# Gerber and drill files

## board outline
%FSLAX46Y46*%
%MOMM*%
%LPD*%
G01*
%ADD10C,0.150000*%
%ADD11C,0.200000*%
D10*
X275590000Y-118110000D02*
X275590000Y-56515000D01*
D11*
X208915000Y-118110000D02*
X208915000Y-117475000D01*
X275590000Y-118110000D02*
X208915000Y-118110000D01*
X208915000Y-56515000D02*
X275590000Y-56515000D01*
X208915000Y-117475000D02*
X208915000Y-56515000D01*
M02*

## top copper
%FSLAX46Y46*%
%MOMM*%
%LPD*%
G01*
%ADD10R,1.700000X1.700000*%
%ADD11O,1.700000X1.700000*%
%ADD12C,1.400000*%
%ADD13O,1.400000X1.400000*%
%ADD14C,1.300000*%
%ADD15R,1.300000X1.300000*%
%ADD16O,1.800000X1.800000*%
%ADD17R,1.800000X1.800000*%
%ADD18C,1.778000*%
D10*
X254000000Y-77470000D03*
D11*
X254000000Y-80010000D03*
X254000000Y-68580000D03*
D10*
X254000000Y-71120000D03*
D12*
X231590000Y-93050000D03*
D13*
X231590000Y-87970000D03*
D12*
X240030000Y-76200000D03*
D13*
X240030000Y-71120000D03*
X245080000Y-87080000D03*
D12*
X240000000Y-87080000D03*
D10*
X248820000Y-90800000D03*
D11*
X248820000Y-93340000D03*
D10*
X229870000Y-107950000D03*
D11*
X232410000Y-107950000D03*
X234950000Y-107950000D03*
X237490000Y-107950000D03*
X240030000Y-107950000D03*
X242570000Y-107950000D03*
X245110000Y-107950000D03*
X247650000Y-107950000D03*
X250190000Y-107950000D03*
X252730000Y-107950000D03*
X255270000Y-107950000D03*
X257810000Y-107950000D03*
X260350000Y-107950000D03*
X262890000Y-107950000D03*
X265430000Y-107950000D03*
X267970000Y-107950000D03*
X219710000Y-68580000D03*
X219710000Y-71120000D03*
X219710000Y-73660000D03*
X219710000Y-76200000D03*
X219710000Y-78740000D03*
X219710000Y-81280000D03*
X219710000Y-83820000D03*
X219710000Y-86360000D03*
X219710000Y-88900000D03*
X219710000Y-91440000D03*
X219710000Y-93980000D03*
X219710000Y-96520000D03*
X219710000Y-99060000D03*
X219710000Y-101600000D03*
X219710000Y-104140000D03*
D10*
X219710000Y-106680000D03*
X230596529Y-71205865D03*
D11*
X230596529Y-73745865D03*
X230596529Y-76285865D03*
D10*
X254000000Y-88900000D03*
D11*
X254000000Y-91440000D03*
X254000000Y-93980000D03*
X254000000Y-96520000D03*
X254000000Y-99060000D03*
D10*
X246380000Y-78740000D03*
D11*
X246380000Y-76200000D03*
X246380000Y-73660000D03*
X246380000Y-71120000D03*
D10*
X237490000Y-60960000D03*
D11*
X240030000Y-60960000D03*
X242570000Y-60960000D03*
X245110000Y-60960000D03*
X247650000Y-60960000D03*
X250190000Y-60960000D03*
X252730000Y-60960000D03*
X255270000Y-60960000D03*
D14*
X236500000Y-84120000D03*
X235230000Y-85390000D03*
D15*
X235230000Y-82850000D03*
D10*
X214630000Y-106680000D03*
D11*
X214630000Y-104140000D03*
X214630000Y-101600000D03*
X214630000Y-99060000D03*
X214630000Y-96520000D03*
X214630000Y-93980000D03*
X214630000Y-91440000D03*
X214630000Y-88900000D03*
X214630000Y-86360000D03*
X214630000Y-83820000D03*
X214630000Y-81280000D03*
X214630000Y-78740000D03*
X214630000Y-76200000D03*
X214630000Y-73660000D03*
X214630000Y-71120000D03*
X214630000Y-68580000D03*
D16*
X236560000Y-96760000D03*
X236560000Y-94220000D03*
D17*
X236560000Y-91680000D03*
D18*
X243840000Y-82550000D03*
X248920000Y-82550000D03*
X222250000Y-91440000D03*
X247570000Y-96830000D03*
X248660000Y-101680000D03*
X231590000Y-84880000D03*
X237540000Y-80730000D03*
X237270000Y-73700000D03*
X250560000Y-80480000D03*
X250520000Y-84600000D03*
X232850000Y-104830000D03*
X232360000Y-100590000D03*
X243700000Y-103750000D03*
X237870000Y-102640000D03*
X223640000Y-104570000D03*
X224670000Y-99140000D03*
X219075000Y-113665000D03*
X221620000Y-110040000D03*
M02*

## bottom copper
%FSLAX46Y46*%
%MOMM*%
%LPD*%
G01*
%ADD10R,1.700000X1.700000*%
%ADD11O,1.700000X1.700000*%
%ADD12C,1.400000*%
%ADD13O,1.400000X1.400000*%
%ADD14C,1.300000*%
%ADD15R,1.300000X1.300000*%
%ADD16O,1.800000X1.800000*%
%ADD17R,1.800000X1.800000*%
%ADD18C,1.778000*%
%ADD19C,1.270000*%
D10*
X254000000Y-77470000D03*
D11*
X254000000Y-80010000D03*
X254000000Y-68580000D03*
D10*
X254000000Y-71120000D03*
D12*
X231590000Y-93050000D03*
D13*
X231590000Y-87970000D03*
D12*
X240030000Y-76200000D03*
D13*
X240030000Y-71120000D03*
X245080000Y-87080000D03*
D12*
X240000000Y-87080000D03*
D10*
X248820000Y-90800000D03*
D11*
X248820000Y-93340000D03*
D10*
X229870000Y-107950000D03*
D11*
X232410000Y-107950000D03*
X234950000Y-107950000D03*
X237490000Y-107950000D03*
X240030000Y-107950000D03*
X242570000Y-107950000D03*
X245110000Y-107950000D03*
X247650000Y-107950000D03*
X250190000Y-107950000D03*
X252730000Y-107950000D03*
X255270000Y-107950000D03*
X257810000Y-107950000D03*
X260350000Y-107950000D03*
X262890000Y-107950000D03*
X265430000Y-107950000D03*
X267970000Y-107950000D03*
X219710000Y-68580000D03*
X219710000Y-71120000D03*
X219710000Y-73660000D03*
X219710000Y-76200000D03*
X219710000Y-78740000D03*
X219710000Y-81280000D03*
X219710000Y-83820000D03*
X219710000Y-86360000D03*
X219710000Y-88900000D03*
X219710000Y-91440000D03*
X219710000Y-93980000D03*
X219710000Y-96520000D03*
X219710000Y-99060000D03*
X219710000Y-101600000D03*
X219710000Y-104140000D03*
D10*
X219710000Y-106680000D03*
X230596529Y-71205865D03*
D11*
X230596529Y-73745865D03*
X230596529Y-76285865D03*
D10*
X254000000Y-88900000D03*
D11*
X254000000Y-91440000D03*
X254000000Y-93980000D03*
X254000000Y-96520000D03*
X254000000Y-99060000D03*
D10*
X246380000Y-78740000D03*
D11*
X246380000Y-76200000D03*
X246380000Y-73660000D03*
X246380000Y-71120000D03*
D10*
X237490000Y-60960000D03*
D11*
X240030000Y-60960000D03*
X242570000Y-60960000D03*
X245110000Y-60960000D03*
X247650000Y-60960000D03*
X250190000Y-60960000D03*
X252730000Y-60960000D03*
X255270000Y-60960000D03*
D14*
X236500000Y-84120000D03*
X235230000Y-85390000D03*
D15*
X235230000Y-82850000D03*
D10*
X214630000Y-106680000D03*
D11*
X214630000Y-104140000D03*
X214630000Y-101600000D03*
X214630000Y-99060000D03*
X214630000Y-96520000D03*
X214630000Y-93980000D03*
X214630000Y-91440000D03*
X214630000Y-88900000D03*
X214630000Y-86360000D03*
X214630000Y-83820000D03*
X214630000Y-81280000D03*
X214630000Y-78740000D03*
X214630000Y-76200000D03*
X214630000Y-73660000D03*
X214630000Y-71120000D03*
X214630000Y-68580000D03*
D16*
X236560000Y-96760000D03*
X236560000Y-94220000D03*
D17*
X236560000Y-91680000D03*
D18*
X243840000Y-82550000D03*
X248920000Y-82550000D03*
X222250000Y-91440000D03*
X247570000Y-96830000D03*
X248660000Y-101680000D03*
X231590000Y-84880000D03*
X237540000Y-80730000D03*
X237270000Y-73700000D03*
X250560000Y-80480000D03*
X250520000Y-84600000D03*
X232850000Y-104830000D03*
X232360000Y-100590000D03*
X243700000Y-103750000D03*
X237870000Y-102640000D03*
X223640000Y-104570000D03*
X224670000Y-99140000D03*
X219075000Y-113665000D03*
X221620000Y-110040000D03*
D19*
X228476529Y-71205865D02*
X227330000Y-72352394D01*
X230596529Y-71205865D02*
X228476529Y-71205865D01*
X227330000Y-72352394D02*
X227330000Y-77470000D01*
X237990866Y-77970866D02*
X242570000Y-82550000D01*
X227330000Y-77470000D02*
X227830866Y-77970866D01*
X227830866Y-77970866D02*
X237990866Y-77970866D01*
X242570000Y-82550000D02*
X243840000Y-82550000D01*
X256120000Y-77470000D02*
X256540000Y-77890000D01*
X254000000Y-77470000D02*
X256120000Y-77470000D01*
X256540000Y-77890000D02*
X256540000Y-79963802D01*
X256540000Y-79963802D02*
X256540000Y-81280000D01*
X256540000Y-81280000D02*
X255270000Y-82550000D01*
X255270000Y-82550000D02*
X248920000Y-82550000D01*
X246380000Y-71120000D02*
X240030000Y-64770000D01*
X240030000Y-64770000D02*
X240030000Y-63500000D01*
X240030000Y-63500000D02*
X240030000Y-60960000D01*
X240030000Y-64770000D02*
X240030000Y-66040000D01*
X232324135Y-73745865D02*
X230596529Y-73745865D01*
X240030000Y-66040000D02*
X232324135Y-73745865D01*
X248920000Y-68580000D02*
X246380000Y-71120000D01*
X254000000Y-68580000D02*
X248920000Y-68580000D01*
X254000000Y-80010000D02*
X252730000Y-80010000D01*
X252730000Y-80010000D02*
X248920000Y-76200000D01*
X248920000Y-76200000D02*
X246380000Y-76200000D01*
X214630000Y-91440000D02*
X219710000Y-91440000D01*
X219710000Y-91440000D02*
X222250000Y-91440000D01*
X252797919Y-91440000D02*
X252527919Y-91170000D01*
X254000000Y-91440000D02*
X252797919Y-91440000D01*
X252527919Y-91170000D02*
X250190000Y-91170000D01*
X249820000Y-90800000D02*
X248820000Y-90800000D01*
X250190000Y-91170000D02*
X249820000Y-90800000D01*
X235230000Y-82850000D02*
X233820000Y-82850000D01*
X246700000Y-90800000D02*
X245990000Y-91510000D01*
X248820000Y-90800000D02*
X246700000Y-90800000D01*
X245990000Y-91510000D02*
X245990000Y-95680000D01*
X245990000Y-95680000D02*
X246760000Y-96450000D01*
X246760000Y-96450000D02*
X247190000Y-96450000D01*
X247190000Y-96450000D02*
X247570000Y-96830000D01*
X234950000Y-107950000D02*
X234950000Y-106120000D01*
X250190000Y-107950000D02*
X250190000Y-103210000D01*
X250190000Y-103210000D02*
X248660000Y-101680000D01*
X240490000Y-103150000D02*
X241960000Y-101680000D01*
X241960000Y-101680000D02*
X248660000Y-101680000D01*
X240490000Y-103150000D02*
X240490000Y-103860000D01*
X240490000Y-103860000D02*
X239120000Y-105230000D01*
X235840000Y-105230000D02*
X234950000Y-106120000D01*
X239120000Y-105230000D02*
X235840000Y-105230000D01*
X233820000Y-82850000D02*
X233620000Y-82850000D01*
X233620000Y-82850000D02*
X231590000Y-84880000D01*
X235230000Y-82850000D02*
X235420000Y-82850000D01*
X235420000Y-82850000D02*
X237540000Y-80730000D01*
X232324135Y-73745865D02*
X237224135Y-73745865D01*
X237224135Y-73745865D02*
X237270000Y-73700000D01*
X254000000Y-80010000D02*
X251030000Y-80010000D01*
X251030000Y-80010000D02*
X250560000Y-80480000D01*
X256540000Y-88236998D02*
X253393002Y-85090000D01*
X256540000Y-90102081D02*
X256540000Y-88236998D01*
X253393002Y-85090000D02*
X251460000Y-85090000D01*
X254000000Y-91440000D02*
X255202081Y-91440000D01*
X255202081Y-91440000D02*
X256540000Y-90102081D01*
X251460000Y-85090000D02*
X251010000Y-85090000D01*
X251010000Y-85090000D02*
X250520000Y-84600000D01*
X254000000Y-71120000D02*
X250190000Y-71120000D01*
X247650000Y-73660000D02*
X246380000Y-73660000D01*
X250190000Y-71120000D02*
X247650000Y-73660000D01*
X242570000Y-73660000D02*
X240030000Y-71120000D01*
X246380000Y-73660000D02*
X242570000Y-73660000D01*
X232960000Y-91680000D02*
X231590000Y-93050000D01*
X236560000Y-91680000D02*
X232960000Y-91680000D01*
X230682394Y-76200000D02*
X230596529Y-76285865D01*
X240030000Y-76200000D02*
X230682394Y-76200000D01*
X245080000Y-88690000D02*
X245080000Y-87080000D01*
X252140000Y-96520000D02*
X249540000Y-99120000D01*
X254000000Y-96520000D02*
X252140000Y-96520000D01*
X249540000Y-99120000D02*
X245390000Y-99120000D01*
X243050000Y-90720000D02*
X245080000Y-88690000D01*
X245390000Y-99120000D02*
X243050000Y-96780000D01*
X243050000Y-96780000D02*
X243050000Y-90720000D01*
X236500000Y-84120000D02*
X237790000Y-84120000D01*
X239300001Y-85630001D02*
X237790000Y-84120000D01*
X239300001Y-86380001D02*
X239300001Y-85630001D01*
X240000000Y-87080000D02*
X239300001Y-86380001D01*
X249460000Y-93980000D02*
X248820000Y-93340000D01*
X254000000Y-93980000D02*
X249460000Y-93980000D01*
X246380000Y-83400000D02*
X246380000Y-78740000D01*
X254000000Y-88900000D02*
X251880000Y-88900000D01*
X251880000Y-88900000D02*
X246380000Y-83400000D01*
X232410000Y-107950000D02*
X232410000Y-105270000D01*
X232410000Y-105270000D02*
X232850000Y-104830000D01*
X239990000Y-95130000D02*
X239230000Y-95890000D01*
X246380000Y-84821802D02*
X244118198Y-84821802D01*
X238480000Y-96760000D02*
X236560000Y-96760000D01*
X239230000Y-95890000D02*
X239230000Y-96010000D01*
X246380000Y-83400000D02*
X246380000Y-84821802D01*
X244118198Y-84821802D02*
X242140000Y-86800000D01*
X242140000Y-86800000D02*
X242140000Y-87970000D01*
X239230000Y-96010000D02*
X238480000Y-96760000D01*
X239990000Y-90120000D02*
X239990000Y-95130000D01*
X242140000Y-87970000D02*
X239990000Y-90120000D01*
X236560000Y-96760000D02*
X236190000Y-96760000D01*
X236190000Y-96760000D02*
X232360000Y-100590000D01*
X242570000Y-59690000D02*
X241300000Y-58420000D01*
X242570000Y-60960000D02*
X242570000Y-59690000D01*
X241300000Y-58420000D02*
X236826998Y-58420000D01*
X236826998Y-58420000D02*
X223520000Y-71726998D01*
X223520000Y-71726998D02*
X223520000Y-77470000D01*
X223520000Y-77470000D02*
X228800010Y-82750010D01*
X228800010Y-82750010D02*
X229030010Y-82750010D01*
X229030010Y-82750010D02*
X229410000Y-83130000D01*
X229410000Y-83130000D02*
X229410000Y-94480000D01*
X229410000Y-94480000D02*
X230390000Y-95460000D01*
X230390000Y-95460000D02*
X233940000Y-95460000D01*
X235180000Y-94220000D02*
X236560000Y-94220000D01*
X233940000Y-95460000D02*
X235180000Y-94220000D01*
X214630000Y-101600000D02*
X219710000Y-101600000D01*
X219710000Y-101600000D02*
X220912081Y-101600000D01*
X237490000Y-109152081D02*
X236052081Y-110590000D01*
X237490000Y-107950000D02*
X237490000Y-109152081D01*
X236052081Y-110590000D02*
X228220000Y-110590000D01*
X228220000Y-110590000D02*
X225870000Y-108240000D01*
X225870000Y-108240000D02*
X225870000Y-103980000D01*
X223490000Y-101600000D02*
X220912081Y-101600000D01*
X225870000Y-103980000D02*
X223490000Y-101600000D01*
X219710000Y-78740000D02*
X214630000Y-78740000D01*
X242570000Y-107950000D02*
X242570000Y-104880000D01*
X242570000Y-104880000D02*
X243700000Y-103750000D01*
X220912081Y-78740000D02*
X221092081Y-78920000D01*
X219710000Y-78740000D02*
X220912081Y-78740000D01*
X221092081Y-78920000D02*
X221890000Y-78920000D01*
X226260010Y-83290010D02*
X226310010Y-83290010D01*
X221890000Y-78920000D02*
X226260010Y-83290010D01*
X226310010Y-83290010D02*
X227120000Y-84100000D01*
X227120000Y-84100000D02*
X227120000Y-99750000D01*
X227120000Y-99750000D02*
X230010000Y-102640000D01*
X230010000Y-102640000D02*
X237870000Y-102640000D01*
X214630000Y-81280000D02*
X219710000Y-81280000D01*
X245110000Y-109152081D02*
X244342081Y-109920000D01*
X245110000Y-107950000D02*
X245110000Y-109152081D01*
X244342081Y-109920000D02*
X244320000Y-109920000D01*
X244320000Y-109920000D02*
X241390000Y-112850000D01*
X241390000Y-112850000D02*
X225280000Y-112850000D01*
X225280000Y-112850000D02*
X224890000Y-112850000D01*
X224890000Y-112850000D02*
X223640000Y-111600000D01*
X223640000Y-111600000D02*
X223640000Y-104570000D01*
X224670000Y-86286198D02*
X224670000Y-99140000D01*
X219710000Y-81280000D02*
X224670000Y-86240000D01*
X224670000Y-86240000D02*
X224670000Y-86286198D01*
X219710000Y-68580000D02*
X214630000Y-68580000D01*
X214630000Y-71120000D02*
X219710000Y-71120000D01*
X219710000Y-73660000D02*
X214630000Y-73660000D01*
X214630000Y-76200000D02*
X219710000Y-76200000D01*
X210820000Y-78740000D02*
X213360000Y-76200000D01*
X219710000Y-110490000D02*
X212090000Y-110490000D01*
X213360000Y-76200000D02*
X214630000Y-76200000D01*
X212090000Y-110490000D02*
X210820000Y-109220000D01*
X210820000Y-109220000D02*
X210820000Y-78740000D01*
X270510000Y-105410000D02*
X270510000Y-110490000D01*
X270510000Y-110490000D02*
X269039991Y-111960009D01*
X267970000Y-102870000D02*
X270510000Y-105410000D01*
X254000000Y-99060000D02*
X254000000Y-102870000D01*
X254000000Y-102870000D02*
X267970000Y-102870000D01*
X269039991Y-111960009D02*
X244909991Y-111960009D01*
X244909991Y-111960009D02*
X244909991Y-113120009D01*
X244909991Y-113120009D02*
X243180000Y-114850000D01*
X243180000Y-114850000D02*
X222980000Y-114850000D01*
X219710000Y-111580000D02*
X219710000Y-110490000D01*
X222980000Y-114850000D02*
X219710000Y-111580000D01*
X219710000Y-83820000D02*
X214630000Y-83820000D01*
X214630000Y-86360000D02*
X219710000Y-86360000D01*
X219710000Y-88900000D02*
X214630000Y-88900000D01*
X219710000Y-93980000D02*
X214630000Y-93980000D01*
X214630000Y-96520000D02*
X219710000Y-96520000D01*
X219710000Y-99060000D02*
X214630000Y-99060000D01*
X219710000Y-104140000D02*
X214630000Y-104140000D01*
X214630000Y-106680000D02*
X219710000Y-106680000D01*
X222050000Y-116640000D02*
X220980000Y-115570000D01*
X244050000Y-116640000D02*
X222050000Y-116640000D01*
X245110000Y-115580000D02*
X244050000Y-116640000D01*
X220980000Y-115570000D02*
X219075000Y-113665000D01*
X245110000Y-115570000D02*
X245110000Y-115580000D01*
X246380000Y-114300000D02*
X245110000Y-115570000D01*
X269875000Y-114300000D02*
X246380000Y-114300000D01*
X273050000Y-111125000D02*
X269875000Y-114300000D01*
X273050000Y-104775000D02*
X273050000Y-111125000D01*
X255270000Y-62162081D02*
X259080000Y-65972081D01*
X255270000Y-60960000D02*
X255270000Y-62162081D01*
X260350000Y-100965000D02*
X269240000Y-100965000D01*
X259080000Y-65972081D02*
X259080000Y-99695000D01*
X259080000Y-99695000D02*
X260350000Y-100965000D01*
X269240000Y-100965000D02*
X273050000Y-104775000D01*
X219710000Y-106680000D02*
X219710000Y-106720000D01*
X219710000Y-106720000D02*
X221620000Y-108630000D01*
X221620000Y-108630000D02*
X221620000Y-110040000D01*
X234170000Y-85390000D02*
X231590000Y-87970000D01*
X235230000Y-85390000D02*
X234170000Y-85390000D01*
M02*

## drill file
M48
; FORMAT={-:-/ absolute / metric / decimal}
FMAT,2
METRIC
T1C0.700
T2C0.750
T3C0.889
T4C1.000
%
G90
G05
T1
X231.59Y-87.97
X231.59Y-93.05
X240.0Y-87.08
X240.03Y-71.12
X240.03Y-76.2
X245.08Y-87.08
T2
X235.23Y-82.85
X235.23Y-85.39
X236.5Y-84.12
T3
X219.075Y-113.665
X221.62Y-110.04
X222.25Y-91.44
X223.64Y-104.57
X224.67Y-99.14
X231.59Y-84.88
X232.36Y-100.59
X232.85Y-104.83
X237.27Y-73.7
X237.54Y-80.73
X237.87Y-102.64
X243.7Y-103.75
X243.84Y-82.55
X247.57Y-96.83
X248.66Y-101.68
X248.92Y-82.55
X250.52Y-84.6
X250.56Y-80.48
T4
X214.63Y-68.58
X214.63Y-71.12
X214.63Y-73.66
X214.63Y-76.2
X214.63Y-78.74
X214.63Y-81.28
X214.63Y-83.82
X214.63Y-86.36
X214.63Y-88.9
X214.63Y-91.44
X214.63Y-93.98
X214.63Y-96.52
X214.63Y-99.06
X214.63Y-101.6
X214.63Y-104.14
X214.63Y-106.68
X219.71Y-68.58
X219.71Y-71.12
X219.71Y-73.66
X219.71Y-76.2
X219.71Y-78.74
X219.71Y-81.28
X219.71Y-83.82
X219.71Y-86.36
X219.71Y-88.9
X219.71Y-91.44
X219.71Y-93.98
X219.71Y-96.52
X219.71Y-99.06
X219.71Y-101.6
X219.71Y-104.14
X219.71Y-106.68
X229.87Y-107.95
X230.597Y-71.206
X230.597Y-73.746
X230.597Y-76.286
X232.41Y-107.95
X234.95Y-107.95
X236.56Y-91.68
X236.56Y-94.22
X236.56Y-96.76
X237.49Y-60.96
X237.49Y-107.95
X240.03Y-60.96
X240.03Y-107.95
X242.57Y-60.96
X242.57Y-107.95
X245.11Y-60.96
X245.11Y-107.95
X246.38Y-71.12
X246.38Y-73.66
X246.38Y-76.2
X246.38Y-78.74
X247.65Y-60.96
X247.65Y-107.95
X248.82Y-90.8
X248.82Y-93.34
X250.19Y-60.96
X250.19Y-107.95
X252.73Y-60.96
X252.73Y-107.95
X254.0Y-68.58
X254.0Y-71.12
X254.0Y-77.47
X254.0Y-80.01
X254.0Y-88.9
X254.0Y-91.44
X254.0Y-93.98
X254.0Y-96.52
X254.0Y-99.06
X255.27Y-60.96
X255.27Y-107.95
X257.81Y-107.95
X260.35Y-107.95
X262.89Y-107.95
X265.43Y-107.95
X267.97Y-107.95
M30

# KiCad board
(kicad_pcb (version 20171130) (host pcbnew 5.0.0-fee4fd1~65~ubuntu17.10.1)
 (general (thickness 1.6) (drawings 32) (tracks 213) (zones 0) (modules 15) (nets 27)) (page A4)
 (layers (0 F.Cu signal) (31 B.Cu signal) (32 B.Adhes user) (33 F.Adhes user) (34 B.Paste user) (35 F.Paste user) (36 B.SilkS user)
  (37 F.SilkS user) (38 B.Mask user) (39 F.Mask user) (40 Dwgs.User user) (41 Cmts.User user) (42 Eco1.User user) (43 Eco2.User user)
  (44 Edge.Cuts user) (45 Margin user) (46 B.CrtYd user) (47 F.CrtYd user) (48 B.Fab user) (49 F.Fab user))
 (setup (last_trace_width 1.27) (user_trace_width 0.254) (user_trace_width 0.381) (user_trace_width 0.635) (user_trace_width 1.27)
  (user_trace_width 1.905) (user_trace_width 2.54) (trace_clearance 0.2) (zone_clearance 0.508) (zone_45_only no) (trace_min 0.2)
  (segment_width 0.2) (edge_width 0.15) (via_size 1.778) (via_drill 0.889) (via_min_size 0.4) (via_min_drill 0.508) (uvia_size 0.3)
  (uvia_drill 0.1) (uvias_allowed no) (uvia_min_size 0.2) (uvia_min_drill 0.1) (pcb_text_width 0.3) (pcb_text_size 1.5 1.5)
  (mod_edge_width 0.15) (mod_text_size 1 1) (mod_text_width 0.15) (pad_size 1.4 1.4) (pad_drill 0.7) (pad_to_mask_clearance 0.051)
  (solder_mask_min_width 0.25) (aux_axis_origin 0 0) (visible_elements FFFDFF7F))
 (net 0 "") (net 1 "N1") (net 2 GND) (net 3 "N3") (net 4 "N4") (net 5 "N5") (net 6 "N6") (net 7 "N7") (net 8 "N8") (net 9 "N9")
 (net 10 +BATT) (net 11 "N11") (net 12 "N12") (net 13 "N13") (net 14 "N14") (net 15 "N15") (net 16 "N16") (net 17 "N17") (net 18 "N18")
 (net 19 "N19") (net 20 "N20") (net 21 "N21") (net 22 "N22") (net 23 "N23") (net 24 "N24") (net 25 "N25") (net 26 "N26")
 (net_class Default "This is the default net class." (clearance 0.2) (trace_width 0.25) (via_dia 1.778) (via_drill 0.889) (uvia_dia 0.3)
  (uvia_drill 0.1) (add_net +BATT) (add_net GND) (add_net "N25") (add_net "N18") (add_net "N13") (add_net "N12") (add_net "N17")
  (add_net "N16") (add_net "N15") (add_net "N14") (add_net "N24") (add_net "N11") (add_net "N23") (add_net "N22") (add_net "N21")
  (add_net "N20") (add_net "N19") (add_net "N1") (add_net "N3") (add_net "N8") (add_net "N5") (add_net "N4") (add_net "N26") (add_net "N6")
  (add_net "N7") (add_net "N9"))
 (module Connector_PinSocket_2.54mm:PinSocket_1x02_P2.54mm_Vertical (layer F.Cu) (at 254 77.47)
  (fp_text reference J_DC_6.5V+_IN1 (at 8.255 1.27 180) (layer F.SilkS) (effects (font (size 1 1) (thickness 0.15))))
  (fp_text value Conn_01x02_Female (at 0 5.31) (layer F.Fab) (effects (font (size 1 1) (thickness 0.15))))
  (pad 1 thru_hole rect (at 0 0) (size 1.7 1.7) (drill 1) (layers *.Cu *.Mask) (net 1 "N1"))
  (pad 2 thru_hole oval (at 0 2.54) (size 1.7 1.7) (drill 1) (layers *.Cu *.Mask) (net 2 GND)))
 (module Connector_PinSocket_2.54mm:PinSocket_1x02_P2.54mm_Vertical (layer F.Cu) (at 254 71.12 180)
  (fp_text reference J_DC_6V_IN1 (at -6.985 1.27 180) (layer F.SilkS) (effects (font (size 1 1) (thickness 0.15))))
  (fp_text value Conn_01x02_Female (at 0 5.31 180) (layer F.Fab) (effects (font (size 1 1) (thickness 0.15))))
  (pad 2 thru_hole oval (at 0 2.54 180) (size 1.7 1.7) (drill 1) (layers *.Cu *.Mask) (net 2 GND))
  (pad 1 thru_hole rect (at 0 0 180) (size 1.7 1.7) (drill 1) (layers *.Cu *.Mask) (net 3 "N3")))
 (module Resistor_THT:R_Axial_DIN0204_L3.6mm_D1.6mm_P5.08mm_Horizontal (layer F.Cu) (at 231.59 93.05 90)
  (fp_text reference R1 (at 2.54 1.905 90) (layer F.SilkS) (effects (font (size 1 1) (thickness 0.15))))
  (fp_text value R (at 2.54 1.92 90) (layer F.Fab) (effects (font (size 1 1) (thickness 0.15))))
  (pad 1 thru_hole circle (at 0 0 90) (size 1.4 1.4) (drill 0.7) (layers *.Cu *.Mask) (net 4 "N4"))
  (pad 2 thru_hole oval (at 5.08 0 90) (size 1.4 1.4) (drill 0.7) (layers *.Cu *.Mask) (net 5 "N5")))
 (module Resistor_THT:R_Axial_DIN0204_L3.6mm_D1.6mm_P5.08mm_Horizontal (layer F.Cu) (at 240.03 76.2 90)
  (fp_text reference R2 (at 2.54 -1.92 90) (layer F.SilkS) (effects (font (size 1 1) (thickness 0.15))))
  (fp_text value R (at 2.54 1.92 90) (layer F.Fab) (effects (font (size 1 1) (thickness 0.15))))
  (pad 1 thru_hole circle (at 0 0 90) (size 1.4 1.4) (drill 0.7) (layers *.Cu *.Mask) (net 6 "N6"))
  (pad 2 thru_hole oval (at 5.08 0 90) (size 1.4 1.4) (drill 0.7) (layers *.Cu *.Mask) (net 3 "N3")))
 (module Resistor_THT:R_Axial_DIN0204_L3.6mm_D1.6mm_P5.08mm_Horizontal (layer F.Cu) (at 240 87.08)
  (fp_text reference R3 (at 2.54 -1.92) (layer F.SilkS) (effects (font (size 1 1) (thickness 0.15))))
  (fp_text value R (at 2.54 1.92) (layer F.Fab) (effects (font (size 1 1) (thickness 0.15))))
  (pad 2 thru_hole oval (at 5.08 0) (size 1.4 1.4) (drill 0.7) (layers *.Cu *.Mask) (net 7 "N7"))
  (pad 1 thru_hole circle (at 0 0) (size 1.4 1.4) (drill 0.7) (layers *.Cu *.Mask) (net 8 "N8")))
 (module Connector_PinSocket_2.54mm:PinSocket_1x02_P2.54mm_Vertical (layer F.Cu) (at 248.82 90.8)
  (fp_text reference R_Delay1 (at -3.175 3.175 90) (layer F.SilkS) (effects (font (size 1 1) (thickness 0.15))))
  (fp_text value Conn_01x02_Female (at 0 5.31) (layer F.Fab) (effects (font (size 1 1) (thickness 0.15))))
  (pad 1 thru_hole rect (at 0 0) (size 1.7 1.7) (drill 1) (layers *.Cu *.Mask) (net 2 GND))
  (pad 2 thru_hole oval (at 0 2.54) (size 1.7 1.7) (drill 1) (layers *.Cu *.Mask) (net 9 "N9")))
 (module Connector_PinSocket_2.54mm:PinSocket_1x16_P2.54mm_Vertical (layer F.Cu) (at 229.87 107.95 90)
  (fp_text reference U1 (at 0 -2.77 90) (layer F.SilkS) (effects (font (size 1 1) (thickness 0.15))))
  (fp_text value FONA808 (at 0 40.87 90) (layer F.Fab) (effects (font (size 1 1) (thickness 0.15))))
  (pad 1 thru_hole rect (at 0 0 90) (size 1.7 1.7) (drill 1) (layers *.Cu *.Mask))
  (pad 2 thru_hole oval (at 0 2.54 90) (size 1.7 1.7) (drill 1) (layers *.Cu *.Mask) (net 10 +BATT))
  (pad 3 thru_hole oval (at 0 5.08 90) (size 1.7 1.7) (drill 1) (layers *.Cu *.Mask) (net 2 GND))
  (pad 4 thru_hole oval (at 0 7.62 90) (size 1.7 1.7) (drill 1) (layers *.Cu *.Mask) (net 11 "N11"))
  (pad 5 thru_hole oval (at 0 10.16 90) (size 1.7 1.7) (drill 1) (layers *.Cu *.Mask))
  (pad 6 thru_hole oval (at 0 12.7 90) (size 1.7 1.7) (drill 1) (layers *.Cu *.Mask) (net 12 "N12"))
  (pad 7 thru_hole oval (at 0 15.24 90) (size 1.7 1.7) (drill 1) (layers *.Cu *.Mask) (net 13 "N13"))
  (pad 8 thru_hole oval (at 0 17.78 90) (size 1.7 1.7) (drill 1) (layers *.Cu *.Mask))
  (pad 9 thru_hole oval (at 0 20.32 90) (size 1.7 1.7) (drill 1) (layers *.Cu *.Mask) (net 2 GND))
  (pad 10 thru_hole oval (at 0 22.86 90) (size 1.7 1.7) (drill 1) (layers *.Cu *.Mask))
  (pad 11 thru_hole oval (at 0 25.4 90) (size 1.7 1.7) (drill 1) (layers *.Cu *.Mask))
  (pad 12 thru_hole oval (at 0 27.94 90) (size 1.7 1.7) (drill 1) (layers *.Cu *.Mask))
  (pad 13 thru_hole oval (at 0 30.48 90) (size 1.7 1.7) (drill 1) (layers *.Cu *.Mask))
  (pad 14 thru_hole oval (at 0 33.02 90) (size 1.7 1.7) (drill 1) (layers *.Cu *.Mask))
  (pad 15 thru_hole oval (at 0 35.56 90) (size 1.7 1.7) (drill 1) (layers *.Cu *.Mask))
  (pad 16 thru_hole oval (at 0 38.1 90) (size 1.7 1.7) (drill 1) (layers *.Cu *.Mask)))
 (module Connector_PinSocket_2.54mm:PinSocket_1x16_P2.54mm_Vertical (layer F.Cu) (at 219.71 106.68 180)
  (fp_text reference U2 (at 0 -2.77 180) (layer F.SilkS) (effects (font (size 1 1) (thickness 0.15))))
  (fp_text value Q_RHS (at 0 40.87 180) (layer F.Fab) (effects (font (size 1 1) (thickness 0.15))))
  (pad 16 thru_hole oval (at 0 38.1 180) (size 1.7 1.7) (drill 1) (layers *.Cu *.Mask) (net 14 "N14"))
  (pad 15 thru_hole oval (at 0 35.56 180) (size 1.7 1.7) (drill 1) (layers *.Cu *.Mask) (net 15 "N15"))
  (pad 14 thru_hole oval (at 0 33.02 180) (size 1.7 1.7) (drill 1) (layers *.Cu *.Mask) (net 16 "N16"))
  (pad 13 thru_hole oval (at 0 30.48 180) (size 1.7 1.7) (drill 1) (layers *.Cu *.Mask) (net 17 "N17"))
  (pad 12 thru_hole oval (at 0 27.94 180) (size 1.7 1.7) (drill 1) (layers *.Cu *.Mask) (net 12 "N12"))
  (pad 11 thru_hole oval (at 0 25.4 180) (size 1.7 1.7) (drill 1) (layers *.Cu *.Mask) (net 13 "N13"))
  (pad 10 thru_hole oval (at 0 22.86 180) (size 1.7 1.7) (drill 1) (layers *.Cu *.Mask) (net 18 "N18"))
  (pad 9 thru_hole oval (at 0 20.32 180) (size 1.7 1.7) (drill 1) (layers *.Cu *.Mask) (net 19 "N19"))
  (pad 8 thru_hole oval (at 0 17.78 180) (size 1.7 1.7) (drill 1) (layers *.Cu *.Mask) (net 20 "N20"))
  (pad 7 thru_hole oval (at 0 15.24 180) (size 1.7 1.7) (drill 1) (layers *.Cu *.Mask) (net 2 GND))
  (pad 6 thru_hole oval (at 0 12.7 180) (size 1.7 1.7) (drill 1) (layers *.Cu *.Mask) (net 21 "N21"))
  (pad 5 thru_hole oval (at 0 10.16 180) (size 1.7 1.7) (drill 1) (layers *.Cu *.Mask) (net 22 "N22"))
  (pad 4 thru_hole oval (at 0 7.62 180) (size 1.7 1.7) (drill 1) (layers *.Cu *.Mask) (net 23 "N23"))
  (pad 3 thru_hole oval (at 0 5.08 180) (size 1.7 1.7) (drill 1) (layers *.Cu *.Mask) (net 11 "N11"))
  (pad 2 thru_hole oval (at 0 2.54 180) (size 1.7 1.7) (drill 1) (layers *.Cu *.Mask) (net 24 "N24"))
  (pad 1 thru_hole rect (at 0 0 180) (size 1.7 1.7) (drill 1) (layers *.Cu *.Mask) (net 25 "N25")))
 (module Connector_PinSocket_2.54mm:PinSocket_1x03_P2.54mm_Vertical (layer F.Cu) (at 230.596529 71.205865)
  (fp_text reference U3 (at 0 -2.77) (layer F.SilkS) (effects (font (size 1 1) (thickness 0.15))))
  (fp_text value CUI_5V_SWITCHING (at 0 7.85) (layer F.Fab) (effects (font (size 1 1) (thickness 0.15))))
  (pad 1 thru_hole rect (at 0 0) (size 1.7 1.7) (drill 1) (layers *.Cu *.Mask) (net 1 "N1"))
  (pad 2 thru_hole oval (at 0 2.54) (size 1.7 1.7) (drill 1) (layers *.Cu *.Mask) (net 2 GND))
  (pad 3 thru_hole oval (at 0 5.08) (size 1.7 1.7) (drill 1) (layers *.Cu *.Mask) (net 6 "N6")))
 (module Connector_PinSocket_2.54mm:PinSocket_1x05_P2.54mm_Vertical (layer F.Cu) (at 254 88.9)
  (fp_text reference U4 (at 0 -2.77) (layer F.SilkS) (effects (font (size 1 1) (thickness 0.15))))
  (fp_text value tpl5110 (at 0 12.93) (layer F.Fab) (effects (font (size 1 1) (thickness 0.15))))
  (pad 1 thru_hole rect (at 0 0) (size 1.7 1.7) (drill 1) (layers *.Cu *.Mask) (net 10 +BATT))
  (pad 2 thru_hole oval (at 0 2.54) (size 1.7 1.7) (drill 1) (layers *.Cu *.Mask) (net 2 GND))
  (pad 3 thru_hole oval (at 0 5.08) (size 1.7 1.7) (drill 1) (layers *.Cu *.Mask) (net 9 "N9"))
  (pad 4 thru_hole oval (at 0 7.62) (size 1.7 1.7) (drill 1) (layers *.Cu *.Mask) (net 7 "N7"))
  (pad 5 thru_hole oval (at 0 10.16) (size 1.7 1.7) (drill 1) (layers *.Cu *.Mask) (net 17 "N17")))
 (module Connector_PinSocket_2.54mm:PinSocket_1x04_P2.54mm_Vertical (layer F.Cu) (at 246.38 78.74 180)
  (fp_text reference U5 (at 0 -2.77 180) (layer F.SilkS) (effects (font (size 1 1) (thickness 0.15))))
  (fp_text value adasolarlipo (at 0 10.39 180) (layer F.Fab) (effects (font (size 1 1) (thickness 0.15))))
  (pad 1 thru_hole rect (at 0 0 180) (size 1.7 1.7) (drill 1) (layers *.Cu *.Mask) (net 10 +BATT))
  (pad 2 thru_hole oval (at 0 2.54 180) (size 1.7 1.7) (drill 1) (layers *.Cu *.Mask) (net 2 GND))
  (pad 3 thru_hole oval (at 0 5.08 180) (size 1.7 1.7) (drill 1) (layers *.Cu *.Mask) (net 3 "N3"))
  (pad 4 thru_hole oval (at 0 7.62 180) (size 1.7 1.7) (drill 1) (layers *.Cu *.Mask) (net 2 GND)))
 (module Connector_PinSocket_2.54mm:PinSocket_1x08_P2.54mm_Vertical (layer F.Cu) (at 237.49 60.96 90)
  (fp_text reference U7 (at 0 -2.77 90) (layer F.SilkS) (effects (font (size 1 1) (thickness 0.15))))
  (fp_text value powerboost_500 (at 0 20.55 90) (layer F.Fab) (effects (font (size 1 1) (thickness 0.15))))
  (pad 1 thru_hole rect (at 0 0 90) (size 1.7 1.7) (drill 1) (layers *.Cu *.Mask))
  (pad 2 thru_hole oval (at 0 2.54 90) (size 1.7 1.7) (drill 1) (layers *.Cu *.Mask) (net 2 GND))
  (pad 3 thru_hole oval (at 0 5.08 90) (size 1.7 1.7) (drill 1) (layers *.Cu *.Mask) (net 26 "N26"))
  (pad 4 thru_hole oval (at 0 7.62 90) (size 1.7 1.7) (drill 1) (layers *.Cu *.Mask))
  (pad 5 thru_hole oval (at 0 10.16 90) (size 1.7 1.7) (drill 1) (layers *.Cu *.Mask))
  (pad 6 thru_hole oval (at 0 12.7 90) (size 1.7 1.7) (drill 1) (layers *.Cu *.Mask))
  (pad 7 thru_hole oval (at 0 15.24 90) (size 1.7 1.7) (drill 1) (layers *.Cu *.Mask))
  (pad 8 thru_hole oval (at 0 17.78 90) (size 1.7 1.7) (drill 1) (layers *.Cu *.Mask) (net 25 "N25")))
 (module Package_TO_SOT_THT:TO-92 (layer F.Cu) (at 235.23 82.85 270)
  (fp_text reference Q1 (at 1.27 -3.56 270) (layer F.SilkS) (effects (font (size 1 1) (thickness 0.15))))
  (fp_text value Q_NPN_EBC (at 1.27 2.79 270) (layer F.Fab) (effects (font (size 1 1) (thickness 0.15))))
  (pad 2 thru_hole circle (at 1.27 -1.27) (size 1.3 1.3) (drill 0.75) (layers *.Cu *.Mask) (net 8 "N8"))
  (pad 3 thru_hole circle (at 2.54 0) (size 1.3 1.3) (drill 0.75) (layers *.Cu *.Mask) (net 5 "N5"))
  (pad 1 thru_hole rect (at 0 0) (size 1.3 1.3) (drill 0.75) (layers *.Cu *.Mask) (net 2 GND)))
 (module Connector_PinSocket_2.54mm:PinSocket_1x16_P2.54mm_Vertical (layer F.Cu) (at 214.63 106.68 180)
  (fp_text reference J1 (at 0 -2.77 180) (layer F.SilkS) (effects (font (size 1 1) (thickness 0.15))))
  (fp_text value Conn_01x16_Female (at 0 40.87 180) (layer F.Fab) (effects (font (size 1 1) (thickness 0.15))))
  (pad 1 thru_hole rect (at 0 0 180) (size 1.7 1.7) (drill 1) (layers *.Cu *.Mask) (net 25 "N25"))
  (pad 2 thru_hole oval (at 0 2.54 180) (size 1.7 1.7) (drill 1) (layers *.Cu *.Mask) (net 24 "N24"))
  (pad 3 thru_hole oval (at 0 5.08 180) (size 1.7 1.7) (drill 1) (layers *.Cu *.Mask) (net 11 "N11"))
  (pad 4 thru_hole oval (at 0 7.62 180) (size 1.7 1.7) (drill 1) (layers *.Cu *.Mask) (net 23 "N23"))
  (pad 5 thru_hole oval (at 0 10.16 180) (size 1.7 1.7) (drill 1) (layers *.Cu *.Mask) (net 22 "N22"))
  (pad 6 thru_hole oval (at 0 12.7 180) (size 1.7 1.7) (drill 1) (layers *.Cu *.Mask) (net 21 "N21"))
  (pad 7 thru_hole oval (at 0 15.24 180) (size 1.7 1.7) (drill 1) (layers *.Cu *.Mask) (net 2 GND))
  (pad 8 thru_hole oval (at 0 17.78 180) (size 1.7 1.7) (drill 1) (layers *.Cu *.Mask) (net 20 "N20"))
  (pad 9 thru_hole oval (at 0 20.32 180) (size 1.7 1.7) (drill 1) (layers *.Cu *.Mask) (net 19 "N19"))
  (pad 10 thru_hole oval (at 0 22.86 180) (size 1.7 1.7) (drill 1) (layers *.Cu *.Mask) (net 18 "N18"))
  (pad 11 thru_hole oval (at 0 25.4 180) (size 1.7 1.7) (drill 1) (layers *.Cu *.Mask) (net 13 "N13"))
  (pad 12 thru_hole oval (at 0 27.94 180) (size 1.7 1.7) (drill 1) (layers *.Cu *.Mask) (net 12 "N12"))
  (pad 13 thru_hole oval (at 0 30.48 180) (size 1.7 1.7) (drill 1) (layers *.Cu *.Mask) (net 17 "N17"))
  (pad 14 thru_hole oval (at 0 33.02 180) (size 1.7 1.7) (drill 1) (layers *.Cu *.Mask) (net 16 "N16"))
  (pad 15 thru_hole oval (at 0 35.56 180) (size 1.7 1.7) (drill 1) (layers *.Cu *.Mask) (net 15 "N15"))
  (pad 16 thru_hole oval (at 0 38.1 180) (size 1.7 1.7) (drill 1) (layers *.Cu *.Mask) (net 14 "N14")))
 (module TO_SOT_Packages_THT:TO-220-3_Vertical (layer F.Cu) (at 236.56 91.68 270)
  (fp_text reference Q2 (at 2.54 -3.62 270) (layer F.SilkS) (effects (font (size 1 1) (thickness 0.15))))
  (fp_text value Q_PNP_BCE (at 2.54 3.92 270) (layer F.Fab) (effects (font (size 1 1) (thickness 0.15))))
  (pad 3 thru_hole oval (at 5.08 0 270) (size 1.8 1.8) (drill 1) (layers *.Cu *.Mask) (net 10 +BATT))
  (pad 2 thru_hole oval (at 2.54 0 270) (size 1.8 1.8) (drill 1) (layers *.Cu *.Mask) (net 26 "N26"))
  (pad 1 thru_hole rect (at 0 0 270) (size 1.8 1.8) (drill 1) (layers *.Cu *.Mask) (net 4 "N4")))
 (gr_line (start 275.59 118.11) (end 275.59 56.515) (layer Edge.Cuts) (width 0.15))
 (gr_line (start 208.915 118.11) (end 208.915 117.475) (layer Edge.Cuts) (width 0.2))
 (gr_line (start 275.59 118.11) (end 208.915 118.11) (layer Edge.Cuts) (width 0.2))
 (gr_line (start 208.915 56.515) (end 275.59 56.515) (layer Edge.Cuts) (width 0.2))
 (gr_line (start 208.915 117.475) (end 208.915 56.515) (layer Edge.Cuts) (width 0.2))
 (segment (start 228.476529 71.205865) (end 227.33 72.352394) (width 1.27) (layer B.Cu) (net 1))
 (segment (start 230.596529 71.205865) (end 228.476529 71.205865) (width 1.27) (layer B.Cu) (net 1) (status 10))
 (segment (start 227.33 72.352394) (end 227.33 77.47) (width 1.27) (layer B.Cu) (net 1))
 (segment (start 237.990866 77.970866) (end 242.57 82.55) (width 1.27) (layer B.Cu) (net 1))
 (segment (start 227.33 77.47) (end 227.830866 77.970866) (width 1.27) (layer B.Cu) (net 1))
 (segment (start 227.830866 77.970866) (end 237.990866 77.970866) (width 1.27) (layer B.Cu) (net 1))
 (via (at 243.84 82.55) (size 1.778) (drill 0.889) (layers F.Cu B.Cu) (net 1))
 (segment (start 242.57 82.55) (end 243.84 82.55) (width 1.27) (layer B.Cu) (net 1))
 (segment (start 256.12 77.47) (end 256.54 77.89) (width 1.27) (layer B.Cu) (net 1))
 (segment (start 254 77.47) (end 256.12 77.47) (width 1.27) (layer B.Cu) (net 1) (status 10))
 (segment (start 256.54 77.89) (end 256.54 79.963802) (width 1.27) (layer B.Cu) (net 1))
 (segment (start 256.54 79.963802) (end 256.54 81.28) (width 1.27) (layer B.Cu) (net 1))
 (segment (start 256.54 81.28) (end 255.27 82.55) (width 1.27) (layer B.Cu) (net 1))
 (via (at 248.92 82.55) (size 1.778) (drill 0.889) (layers F.Cu B.Cu) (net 1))
 (segment (start 255.27 82.55) (end 248.92 82.55) (width 1.27) (layer B.Cu) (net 1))
 (segment (start 246.38 71.12) (end 240.03 64.77) (width 1.27) (layer B.Cu) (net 2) (status 10))
 (segment (start 240.03 64.77) (end 240.03 63.5) (width 1.27) (layer B.Cu) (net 2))
 (segment (start 240.03 63.5) (end 240.03 60.96) (width 1.27) (layer B.Cu) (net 2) (status 20))
 (segment (start 240.03 64.77) (end 240.03 66.04) (width 1.27) (layer B.Cu) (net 2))
 (segment (start 232.324135 73.745865) (end 230.596529 73.745865) (width 1.27) (layer B.Cu) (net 2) (status 20))
 (segment (start 240.03 66.04) (end 232.324135 73.745865) (width 1.27) (layer B.Cu) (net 2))
 (segment (start 248.92 68.58) (end 246.38 71.12) (width 1.27) (layer B.Cu) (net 2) (status 20))
 (segment (start 254 68.58) (end 248.92 68.58) (width 1.27) (layer B.Cu) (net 2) (status 10))
 (segment (start 254 80.01) (end 252.73 80.01) (width 1.27) (layer B.Cu) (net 2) (status 10))
 (segment (start 252.73 80.01) (end 248.92 76.2) (width 1.27) (layer B.Cu) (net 2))
 (segment (start 248.92 76.2) (end 246.38 76.2) (width 1.27) (layer B.Cu) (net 2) (status 20))
 (segment (start 214.63 91.44) (end 219.71 91.44) (width 1.27) (layer B.Cu) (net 2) (status 30))
 (via (at 222.25 91.44) (size 1.778) (drill 0.889) (layers F.Cu B.Cu) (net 2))
 (segment (start 219.71 91.44) (end 222.25 91.44) (width 1.27) (layer B.Cu) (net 2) (status 10))
 (segment (start 252.797919 91.44) (end 252.527919 91.17) (width 1.27) (layer B.Cu) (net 2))
 (segment (start 254 91.44) (end 252.797919 91.44) (width 1.27) (layer B.Cu) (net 2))
 (segment (start 252.527919 91.17) (end 250.19 91.17) (width 1.27) (layer B.Cu) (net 2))
 (segment (start 249.82 90.8) (end 248.82 90.8) (width 1.27) (layer B.Cu) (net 2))
 (segment (start 250.19 91.17) (end 249.82 90.8) (width 1.27) (layer B.Cu) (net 2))
 (segment (start 235.23 82.85) (end 233.82 82.85) (width 1.27) (layer B.Cu) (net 2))
 (segment (start 246.7 90.8) (end 245.99 91.51) (width 1.27) (layer B.Cu) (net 2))
 (segment (start 248.82 90.8) (end 246.7 90.8) (width 1.27) (layer B.Cu) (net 2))
 (segment (start 245.99 91.51) (end 245.99 95.68) (width 1.27) (layer B.Cu) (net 2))
 (segment (start 245.99 95.68) (end 246.76 96.45) (width 1.27) (layer B.Cu) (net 2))
 (via (at 247.57 96.83) (size 1.778) (drill 0.889) (layers F.Cu B.Cu) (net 2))
 (segment (start 246.76 96.45) (end 247.19 96.45) (width 1.27) (layer B.Cu) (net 2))
 (segment (start 247.19 96.45) (end 247.57 96.83) (width 1.27) (layer B.Cu) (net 2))
 (segment (start 234.95 107.95) (end 234.95 106.12) (width 1.27) (layer B.Cu) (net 2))
 (segment (start 250.19 107.95) (end 250.19 103.21) (width 1.27) (layer B.Cu) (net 2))
 (segment (start 250.19 103.21) (end 248.66 101.68) (width 1.27) (layer B.Cu) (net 2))
 (segment (start 240.49 103.15) (end 241.96 101.68) (width 1.27) (layer B.Cu) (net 2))
 (segment (start 241.96 101.68) (end 248.66 101.68) (width 1.27) (layer B.Cu) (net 2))
 (via (at 248.66 101.68) (size 1.778) (drill 0.889) (layers F.Cu B.Cu) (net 2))
 (segment (start 240.49 103.15) (end 240.49 103.86) (width 1.27) (layer B.Cu) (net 2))
 (segment (start 240.49 103.86) (end 239.12 105.23) (width 1.27) (layer B.Cu) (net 2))
 (segment (start 235.84 105.23) (end 234.95 106.12) (width 1.27) (layer B.Cu) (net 2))
 (segment (start 239.12 105.23) (end 235.84 105.23) (width 1.27) (layer B.Cu) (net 2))
 (via (at 231.59 84.88) (size 1.778) (drill 0.889) (layers F.Cu B.Cu) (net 2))
 (segment (start 233.82 82.85) (end 233.62 82.85) (width 1.27) (layer B.Cu) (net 2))
 (segment (start 233.62 82.85) (end 231.59 84.88) (width 1.27) (layer B.Cu) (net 2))
 (via (at 237.54 80.73) (size 1.778) (drill 0.889) (layers F.Cu B.Cu) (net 2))
 (segment (start 235.23 82.85) (end 235.42 82.85) (width 1.27) (layer B.Cu) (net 2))
 (segment (start 235.42 82.85) (end 237.54 80.73) (width 1.27) (layer B.Cu) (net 2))
 (segment (start 232.324135 73.745865) (end 237.224135 73.745865) (width 1.27) (layer B.Cu) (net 2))
 (via (at 237.27 73.7) (size 1.778) (drill 0.889) (layers F.Cu B.Cu) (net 2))
 (segment (start 237.224135 73.745865) (end 237.27 73.7) (width 1.27) (layer B.Cu) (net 2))
 (via (at 250.56 80.48) (size 1.778) (drill 0.889) (layers F.Cu B.Cu) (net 2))
 (segment (start 254 80.01) (end 251.03 80.01) (width 1.27) (layer B.Cu) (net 2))
 (segment (start 251.03 80.01) (end 250.56 80.48) (width 1.27) (layer B.Cu) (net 2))
 (segment (start 256.54 88.236998) (end 253.393002 85.09) (width 1.27) (layer B.Cu) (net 2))
 (segment (start 256.54 90.102081) (end 256.54 88.236998) (width 1.27) (layer B.Cu) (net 2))
 (segment (start 253.393002 85.09) (end 251.46 85.09) (width 1.27) (layer B.Cu) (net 2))
 (segment (start 254 91.44) (end 255.202081 91.44) (width 1.27) (layer B.Cu) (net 2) (status 10))
 (segment (start 255.202081 91.44) (end 256.54 90.102081) (width 1.27) (layer B.Cu) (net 2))
 (segment (start 251.46 85.09) (end 251.01 85.09) (width 1.27) (layer B.Cu) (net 2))
 (via (at 250.52 84.6) (size 1.778) (drill 0.889) (layers F.Cu B.Cu) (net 2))
 (segment (start 251.01 85.09) (end 250.52 84.6) (width 1.27) (layer B.Cu) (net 2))
 (segment (start 254 71.12) (end 250.19 71.12) (width 1.27) (layer B.Cu) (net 3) (status 10))
 (segment (start 247.65 73.66) (end 246.38 73.66) (width 1.27) (layer B.Cu) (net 3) (status 20))
 (segment (start 250.19 71.12) (end 247.65 73.66) (width 1.27) (layer B.Cu) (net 3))
 (segment (start 242.57 73.66) (end 240.03 71.12) (width 1.27) (layer B.Cu) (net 3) (status 20))
 (segment (start 246.38 73.66) (end 242.57 73.66) (width 1.27) (layer B.Cu) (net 3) (status 10))
 (segment (start 232.96 91.68) (end 231.59 93.05) (width 1.27) (layer B.Cu) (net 4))
 (segment (start 236.56 91.68) (end 232.96 91.68) (width 1.27) (layer B.Cu) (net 4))
 (segment (start 230.682394 76.2) (end 230.596529 76.285865) (width 1.27) (layer B.Cu) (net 6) (status 30))
 (segment (start 240.03 76.2) (end 230.682394 76.2) (width 1.27) (layer B.Cu) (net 6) (status 30))
 (segment (start 245.08 88.69) (end 245.08 87.08) (width 1.27) (layer B.Cu) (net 7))
 (segment (start 252.14 96.52) (end 249.54 99.12) (width 1.27) (layer B.Cu) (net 7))
 (segment (start 254 96.52) (end 252.14 96.52) (width 1.27) (layer B.Cu) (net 7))
 (segment (start 249.54 99.12) (end 245.39 99.12) (width 1.27) (layer B.Cu) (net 7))
 (segment (start 243.05 90.72) (end 245.08 88.69) (width 1.27) (layer B.Cu) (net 7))
 (segment (start 245.39 99.12) (end 243.05 96.78) (width 1.27) (layer B.Cu) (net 7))
 (segment (start 243.05 96.78) (end 243.05 90.72) (width 1.27) (layer B.Cu) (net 7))
 (segment (start 236.5 84.12) (end 237.79 84.12) (width 1.27) (layer B.Cu) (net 8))
 (segment (start 239.300001 85.630001) (end 237.79 84.12) (width 1.27) (layer B.Cu) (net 8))
 (segment (start 239.300001 86.380001) (end 239.300001 85.630001) (width 1.27) (layer B.Cu) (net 8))
 (segment (start 240 87.08) (end 239.300001 86.380001) (width 1.27) (layer B.Cu) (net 8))
 (segment (start 249.46 93.98) (end 248.82 93.34) (width 1.27) (layer B.Cu) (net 9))
 (segment (start 254 93.98) (end 249.46 93.98) (width 1.27) (layer B.Cu) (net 9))
 (segment (start 246.38 83.4) (end 246.38 78.74) (width 1.27) (layer B.Cu) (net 10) (status 20))
 (segment (start 254 88.9) (end 251.88 88.9) (width 1.27) (layer B.Cu) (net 10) (status 10))
 (segment (start 251.88 88.9) (end 246.38 83.4) (width 1.27) (layer B.Cu) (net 10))
 (via (at 232.85 104.83) (size 1.778) (drill 0.889) (layers F.Cu B.Cu) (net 10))
 (segment (start 232.41 107.95) (end 232.41 105.27) (width 1.27) (layer B.Cu) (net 10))
 (segment (start 232.41 105.27) (end 232.85 104.83) (width 1.27) (layer B.Cu) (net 10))
 (segment (start 239.99 95.13) (end 239.23 95.89) (width 1.27) (layer B.Cu) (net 10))
 (segment (start 246.38 84.821802) (end 244.118198 84.821802) (width 1.27) (layer B.Cu) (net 10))
 (segment (start 238.48 96.76) (end 236.56 96.76) (width 1.27) (layer B.Cu) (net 10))
 (segment (start 239.23 95.89) (end 239.23 96.01) (width 1.27) (layer B.Cu) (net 10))
 (segment (start 246.38 83.4) (end 246.38 84.821802) (width 1.27) (layer B.Cu) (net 10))
 (segment (start 244.118198 84.821802) (end 242.14 86.8) (width 1.27) (layer B.Cu) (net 10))
 (segment (start 242.14 86.8) (end 242.14 87.97) (width 1.27) (layer B.Cu) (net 10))
 (segment (start 239.23 96.01) (end 238.48 96.76) (width 1.27) (layer B.Cu) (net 10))
 (segment (start 239.99 90.12) (end 239.99 95.13) (width 1.27) (layer B.Cu) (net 10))
 (segment (start 242.14 87.97) (end 239.99 90.12) (width 1.27) (layer B.Cu) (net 10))
 (via (at 232.36 100.59) (size 1.778) (drill 0.889) (layers F.Cu B.Cu) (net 10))
 (segment (start 236.56 96.76) (end 236.19 96.76) (width 1.27) (layer B.Cu) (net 10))
 (segment (start 236.19 96.76) (end 232.36 100.59) (width 1.27) (layer B.Cu) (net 10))
 (segment (start 242.57 59.69) (end 241.3 58.42) (width 1.27) (layer B.Cu) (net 26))
 (segment (start 242.57 60.96) (end 242.57 59.69) (width 1.27) (layer B.Cu) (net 26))
 (segment (start 241.3 58.42) (end 236.826998 58.42) (width 1.27) (layer B.Cu) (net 26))
 (segment (start 236.826998 58.42) (end 223.52 71.726998) (width 1.27) (layer B.Cu) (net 26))
 (segment (start 223.52 71.726998) (end 223.52 77.47) (width 1.27) (layer B.Cu) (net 26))
 (segment (start 223.52 77.47) (end 228.80001 82.75001) (width 1.27) (layer B.Cu) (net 26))
 (segment (start 228.80001 82.75001) (end 229.03001 82.75001) (width 1.27) (layer B.Cu) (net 26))
 (segment (start 229.03001 82.75001) (end 229.41 83.13) (width 1.27) (layer B.Cu) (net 26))
 (segment (start 229.41 83.13) (end 229.41 94.48) (width 1.27) (layer B.Cu) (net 26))
 (segment (start 229.41 94.48) (end 230.39 95.46) (width 1.27) (layer B.Cu) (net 26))
 (segment (start 230.39 95.46) (end 233.94 95.46) (width 1.27) (layer B.Cu) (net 26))
 (segment (start 235.18 94.22) (end 236.56 94.22) (width 1.27) (layer B.Cu) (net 26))
 (segment (start 233.94 95.46) (end 235.18 94.22) (width 1.27) (layer B.Cu) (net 26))
 (segment (start 214.63 101.6) (end 219.71 101.6) (width 1.27) (layer B.Cu) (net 11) (status 30))
 (segment (start 219.71 101.6) (end 220.912081 101.6) (width 1.27) (layer B.Cu) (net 11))
 (segment (start 237.49 109.152081) (end 236.052081 110.59) (width 1.27) (layer B.Cu) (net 11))
 (segment (start 237.49 107.95) (end 237.49 109.152081) (width 1.27) (layer B.Cu) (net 11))
 (segment (start 236.052081 110.59) (end 228.22 110.59) (width 1.27) (layer B.Cu) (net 11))
 (segment (start 228.22 110.59) (end 225.87 108.24) (width 1.27) (layer B.Cu) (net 11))
 (segment (start 225.87 108.24) (end 225.87 103.98) (width 1.27) (layer B.Cu) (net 11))
 (segment (start 223.49 101.6) (end 220.912081 101.6) (width 1.27) (layer B.Cu) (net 11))
 (segment (start 225.87 103.98) (end 223.49 101.6) (width 1.27) (layer B.Cu) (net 11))
 (segment (start 219.71 78.74) (end 214.63 78.74) (width 1.27) (layer B.Cu) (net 12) (status 30))
 (via (at 243.7 103.75) (size 1.778) (drill 0.889) (layers F.Cu B.Cu) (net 12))
 (segment (start 242.57 107.95) (end 242.57 104.88) (width 1.27) (layer B.Cu) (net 12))
 (segment (start 242.57 104.88) (end 243.7 103.75) (width 1.27) (layer B.Cu) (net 12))
 (segment (start 220.912081 78.74) (end 221.092081 78.92) (width 1.27) (layer B.Cu) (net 12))
 (segment (start 219.71 78.74) (end 220.912081 78.74) (width 1.27) (layer B.Cu) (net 12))
 (segment (start 221.092081 78.92) (end 221.89 78.92) (width 1.27) (layer B.Cu) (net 12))
 (segment (start 226.26001 83.29001) (end 226.31001 83.29001) (width 1.27) (layer B.Cu) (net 12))
 (segment (start 221.89 78.92) (end 226.26001 83.29001) (width 1.27) (layer B.Cu) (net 12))
 (segment (start 226.31001 83.29001) (end 227.12 84.1) (width 1.27) (layer B.Cu) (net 12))
 (segment (start 227.12 84.1) (end 227.12 99.75) (width 1.27) (layer B.Cu) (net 12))
 (segment (start 227.12 99.75) (end 230.01 102.64) (width 1.27) (layer B.Cu) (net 12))
 (via (at 237.87 102.64) (size 1.778) (drill 0.889) (layers F.Cu B.Cu) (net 12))
 (segment (start 230.01 102.64) (end 237.87 102.64) (width 1.27) (layer B.Cu) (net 12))
 (segment (start 214.63 81.28) (end 219.71 81.28) (width 1.27) (layer B.Cu) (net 13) (status 30))
 (segment (start 245.11 109.152081) (end 244.342081 109.92) (width 1.27) (layer B.Cu) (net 13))
 (segment (start 245.11 107.95) (end 245.11 109.152081) (width 1.27) (layer B.Cu) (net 13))
 (segment (start 244.342081 109.92) (end 244.32 109.92) (width 1.27) (layer B.Cu) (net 13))
 (segment (start 244.32 109.92) (end 241.39 112.85) (width 1.27) (layer B.Cu) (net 13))
 (segment (start 241.39 112.85) (end 225.28 112.85) (width 1.27) (layer B.Cu) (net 13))
 (segment (start 225.28 112.85) (end 224.89 112.85) (width 1.27) (layer B.Cu) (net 13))
 (via (at 223.64 104.57) (size 1.778) (drill 0.889) (layers F.Cu B.Cu) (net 13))
 (segment (start 224.89 112.85) (end 223.64 111.6) (width 1.27) (layer B.Cu) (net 13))
 (segment (start 223.64 111.6) (end 223.64 104.57) (width 1.27) (layer B.Cu) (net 13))
 (via (at 224.67 99.14) (size 1.778) (drill 0.889) (layers F.Cu B.Cu) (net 13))
 (segment (start 224.67 86.286198) (end 224.67 99.14) (width 1.27) (layer B.Cu) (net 13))
 (segment (start 219.71 81.28) (end 224.67 86.24) (width 1.27) (layer B.Cu) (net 13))
 (segment (start 224.67 86.24) (end 224.67 86.286198) (width 1.27) (layer B.Cu) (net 13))
 (segment (start 219.71 68.58) (end 214.63 68.58) (width 1.27) (layer B.Cu) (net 14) (status 30))
 (segment (start 214.63 71.12) (end 219.71 71.12) (width 1.27) (layer B.Cu) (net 15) (status 30))
 (segment (start 219.71 73.66) (end 214.63 73.66) (width 1.27) (layer B.Cu) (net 16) (status 30))
 (segment (start 214.63 76.2) (end 219.71 76.2) (width 1.27) (layer B.Cu) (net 17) (status 30))
 (segment (start 210.82 78.74) (end 213.36 76.2) (width 1.27) (layer B.Cu) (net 17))
 (segment (start 219.71 110.49) (end 212.09 110.49) (width 1.27) (layer B.Cu) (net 17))
 (segment (start 213.36 76.2) (end 214.63 76.2) (width 1.27) (layer B.Cu) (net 17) (status 20))
 (segment (start 212.09 110.49) (end 210.82 109.22) (width 1.27) (layer B.Cu) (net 17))
 (segment (start 210.82 109.22) (end 210.82 78.74) (width 1.27) (layer B.Cu) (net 17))
 (segment (start 270.51 105.41) (end 270.51 110.49) (width 1.27) (layer B.Cu) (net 17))
 (segment (start 270.51 110.49) (end 269.039991 111.960009) (width 1.27) (layer B.Cu) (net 17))
 (segment (start 267.97 102.87) (end 270.51 105.41) (width 1.27) (layer B.Cu) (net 17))
 (segment (start 254 99.06) (end 254 102.87) (width 1.27) (layer B.Cu) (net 17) (status 10))
 (segment (start 254 102.87) (end 267.97 102.87) (width 1.27) (layer B.Cu) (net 17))
 (segment (start 269.039991 111.960009) (end 244.909991 111.960009) (width 1.27) (layer B.Cu) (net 17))
 (segment (start 244.909991 111.960009) (end 244.909991 113.120009) (width 1.27) (layer B.Cu) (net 17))
 (segment (start 244.909991 113.120009) (end 243.18 114.85) (width 1.27) (layer B.Cu) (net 17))
 (segment (start 243.18 114.85) (end 222.98 114.85) (width 1.27) (layer B.Cu) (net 17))
 (segment (start 219.71 111.58) (end 219.71 110.49) (width 1.27) (layer B.Cu) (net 17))
 (segment (start 222.98 114.85) (end 219.71 111.58) (width 1.27) (layer B.Cu) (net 17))
 (segment (start 219.71 83.82) (end 214.63 83.82) (width 1.27) (layer B.Cu) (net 18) (status 30))
 (segment (start 214.63 86.36) (end 219.71 86.36) (width 1.27) (layer B.Cu) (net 19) (status 30))
 (segment (start 219.71 88.9) (end 214.63 88.9) (width 1.27) (layer B.Cu) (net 20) (status 30))
 (segment (start 219.71 93.98) (end 214.63 93.98) (width 1.27) (layer B.Cu) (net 21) (status 30))
 (segment (start 214.63 96.52) (end 219.71 96.52) (width 1.27) (layer B.Cu) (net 22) (status 30))
 (segment (start 219.71 99.06) (end 214.63 99.06) (width 1.27) (layer B.Cu) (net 23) (status 30))
 (segment (start 219.71 104.14) (end 214.63 104.14) (width 1.27) (layer B.Cu) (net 24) (status 30))
 (segment (start 214.63 106.68) (end 219.71 106.68) (width 1.27) (layer B.Cu) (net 25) (status 30))
 (via (at 219.075 113.665) (size 1.778) (drill 0.889) (layers F.Cu B.Cu) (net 25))
 (segment (start 222.05 116.64) (end 220.98 115.57) (width 1.27) (layer B.Cu) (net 25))
 (segment (start 244.05 116.64) (end 222.05 116.64) (width 1.27) (layer B.Cu) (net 25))
 (segment (start 245.11 115.58) (end 244.05 116.64) (width 1.27) (layer B.Cu) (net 25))
 (segment (start 220.98 115.57) (end 219.075 113.665) (width 1.27) (layer B.Cu) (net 25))
 (segment (start 245.11 115.57) (end 245.11 115.58) (width 1.27) (layer B.Cu) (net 25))
 (segment (start 246.38 114.3) (end 245.11 115.57) (width 1.27) (layer B.Cu) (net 25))
 (segment (start 269.875 114.3) (end 246.38 114.3) (width 1.27) (layer B.Cu) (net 25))
 (segment (start 273.05 111.125) (end 269.875 114.3) (width 1.27) (layer B.Cu) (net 25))
 (segment (start 273.05 104.775) (end 273.05 111.125) (width 1.27) (layer B.Cu) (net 25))
 (segment (start 255.27 62.162081) (end 259.08 65.972081) (width 1.27) (layer B.Cu) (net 25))
 (segment (start 255.27 60.96) (end 255.27 62.162081) (width 1.27) (layer B.Cu) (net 25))
 (segment (start 260.35 100.965) (end 269.24 100.965) (width 1.27) (layer B.Cu) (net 25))
 (segment (start 259.08 65.972081) (end 259.08 99.695) (width 1.27) (layer B.Cu) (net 25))
 (segment (start 259.08 99.695) (end 260.35 100.965) (width 1.27) (layer B.Cu) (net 25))
 (segment (start 269.24 100.965) (end 273.05 104.775) (width 1.27) (layer B.Cu) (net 25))
 (segment (start 219.71 106.68) (end 219.71 106.72) (width 1.27) (layer B.Cu) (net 25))
 (via (at 221.62 110.04) (size 1.778) (drill 0.889) (layers F.Cu B.Cu) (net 25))
 (segment (start 219.71 106.72) (end 221.62 108.63) (width 1.27) (layer B.Cu) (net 25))
 (segment (start 221.62 108.63) (end 221.62 110.04) (width 1.27) (layer B.Cu) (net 25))
 (segment (start 234.17 85.39) (end 231.59 87.97) (width 1.27) (layer B.Cu) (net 5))
 (segment (start 235.23 85.39) (end 234.17 85.39) (width 1.27) (layer B.Cu) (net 5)))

